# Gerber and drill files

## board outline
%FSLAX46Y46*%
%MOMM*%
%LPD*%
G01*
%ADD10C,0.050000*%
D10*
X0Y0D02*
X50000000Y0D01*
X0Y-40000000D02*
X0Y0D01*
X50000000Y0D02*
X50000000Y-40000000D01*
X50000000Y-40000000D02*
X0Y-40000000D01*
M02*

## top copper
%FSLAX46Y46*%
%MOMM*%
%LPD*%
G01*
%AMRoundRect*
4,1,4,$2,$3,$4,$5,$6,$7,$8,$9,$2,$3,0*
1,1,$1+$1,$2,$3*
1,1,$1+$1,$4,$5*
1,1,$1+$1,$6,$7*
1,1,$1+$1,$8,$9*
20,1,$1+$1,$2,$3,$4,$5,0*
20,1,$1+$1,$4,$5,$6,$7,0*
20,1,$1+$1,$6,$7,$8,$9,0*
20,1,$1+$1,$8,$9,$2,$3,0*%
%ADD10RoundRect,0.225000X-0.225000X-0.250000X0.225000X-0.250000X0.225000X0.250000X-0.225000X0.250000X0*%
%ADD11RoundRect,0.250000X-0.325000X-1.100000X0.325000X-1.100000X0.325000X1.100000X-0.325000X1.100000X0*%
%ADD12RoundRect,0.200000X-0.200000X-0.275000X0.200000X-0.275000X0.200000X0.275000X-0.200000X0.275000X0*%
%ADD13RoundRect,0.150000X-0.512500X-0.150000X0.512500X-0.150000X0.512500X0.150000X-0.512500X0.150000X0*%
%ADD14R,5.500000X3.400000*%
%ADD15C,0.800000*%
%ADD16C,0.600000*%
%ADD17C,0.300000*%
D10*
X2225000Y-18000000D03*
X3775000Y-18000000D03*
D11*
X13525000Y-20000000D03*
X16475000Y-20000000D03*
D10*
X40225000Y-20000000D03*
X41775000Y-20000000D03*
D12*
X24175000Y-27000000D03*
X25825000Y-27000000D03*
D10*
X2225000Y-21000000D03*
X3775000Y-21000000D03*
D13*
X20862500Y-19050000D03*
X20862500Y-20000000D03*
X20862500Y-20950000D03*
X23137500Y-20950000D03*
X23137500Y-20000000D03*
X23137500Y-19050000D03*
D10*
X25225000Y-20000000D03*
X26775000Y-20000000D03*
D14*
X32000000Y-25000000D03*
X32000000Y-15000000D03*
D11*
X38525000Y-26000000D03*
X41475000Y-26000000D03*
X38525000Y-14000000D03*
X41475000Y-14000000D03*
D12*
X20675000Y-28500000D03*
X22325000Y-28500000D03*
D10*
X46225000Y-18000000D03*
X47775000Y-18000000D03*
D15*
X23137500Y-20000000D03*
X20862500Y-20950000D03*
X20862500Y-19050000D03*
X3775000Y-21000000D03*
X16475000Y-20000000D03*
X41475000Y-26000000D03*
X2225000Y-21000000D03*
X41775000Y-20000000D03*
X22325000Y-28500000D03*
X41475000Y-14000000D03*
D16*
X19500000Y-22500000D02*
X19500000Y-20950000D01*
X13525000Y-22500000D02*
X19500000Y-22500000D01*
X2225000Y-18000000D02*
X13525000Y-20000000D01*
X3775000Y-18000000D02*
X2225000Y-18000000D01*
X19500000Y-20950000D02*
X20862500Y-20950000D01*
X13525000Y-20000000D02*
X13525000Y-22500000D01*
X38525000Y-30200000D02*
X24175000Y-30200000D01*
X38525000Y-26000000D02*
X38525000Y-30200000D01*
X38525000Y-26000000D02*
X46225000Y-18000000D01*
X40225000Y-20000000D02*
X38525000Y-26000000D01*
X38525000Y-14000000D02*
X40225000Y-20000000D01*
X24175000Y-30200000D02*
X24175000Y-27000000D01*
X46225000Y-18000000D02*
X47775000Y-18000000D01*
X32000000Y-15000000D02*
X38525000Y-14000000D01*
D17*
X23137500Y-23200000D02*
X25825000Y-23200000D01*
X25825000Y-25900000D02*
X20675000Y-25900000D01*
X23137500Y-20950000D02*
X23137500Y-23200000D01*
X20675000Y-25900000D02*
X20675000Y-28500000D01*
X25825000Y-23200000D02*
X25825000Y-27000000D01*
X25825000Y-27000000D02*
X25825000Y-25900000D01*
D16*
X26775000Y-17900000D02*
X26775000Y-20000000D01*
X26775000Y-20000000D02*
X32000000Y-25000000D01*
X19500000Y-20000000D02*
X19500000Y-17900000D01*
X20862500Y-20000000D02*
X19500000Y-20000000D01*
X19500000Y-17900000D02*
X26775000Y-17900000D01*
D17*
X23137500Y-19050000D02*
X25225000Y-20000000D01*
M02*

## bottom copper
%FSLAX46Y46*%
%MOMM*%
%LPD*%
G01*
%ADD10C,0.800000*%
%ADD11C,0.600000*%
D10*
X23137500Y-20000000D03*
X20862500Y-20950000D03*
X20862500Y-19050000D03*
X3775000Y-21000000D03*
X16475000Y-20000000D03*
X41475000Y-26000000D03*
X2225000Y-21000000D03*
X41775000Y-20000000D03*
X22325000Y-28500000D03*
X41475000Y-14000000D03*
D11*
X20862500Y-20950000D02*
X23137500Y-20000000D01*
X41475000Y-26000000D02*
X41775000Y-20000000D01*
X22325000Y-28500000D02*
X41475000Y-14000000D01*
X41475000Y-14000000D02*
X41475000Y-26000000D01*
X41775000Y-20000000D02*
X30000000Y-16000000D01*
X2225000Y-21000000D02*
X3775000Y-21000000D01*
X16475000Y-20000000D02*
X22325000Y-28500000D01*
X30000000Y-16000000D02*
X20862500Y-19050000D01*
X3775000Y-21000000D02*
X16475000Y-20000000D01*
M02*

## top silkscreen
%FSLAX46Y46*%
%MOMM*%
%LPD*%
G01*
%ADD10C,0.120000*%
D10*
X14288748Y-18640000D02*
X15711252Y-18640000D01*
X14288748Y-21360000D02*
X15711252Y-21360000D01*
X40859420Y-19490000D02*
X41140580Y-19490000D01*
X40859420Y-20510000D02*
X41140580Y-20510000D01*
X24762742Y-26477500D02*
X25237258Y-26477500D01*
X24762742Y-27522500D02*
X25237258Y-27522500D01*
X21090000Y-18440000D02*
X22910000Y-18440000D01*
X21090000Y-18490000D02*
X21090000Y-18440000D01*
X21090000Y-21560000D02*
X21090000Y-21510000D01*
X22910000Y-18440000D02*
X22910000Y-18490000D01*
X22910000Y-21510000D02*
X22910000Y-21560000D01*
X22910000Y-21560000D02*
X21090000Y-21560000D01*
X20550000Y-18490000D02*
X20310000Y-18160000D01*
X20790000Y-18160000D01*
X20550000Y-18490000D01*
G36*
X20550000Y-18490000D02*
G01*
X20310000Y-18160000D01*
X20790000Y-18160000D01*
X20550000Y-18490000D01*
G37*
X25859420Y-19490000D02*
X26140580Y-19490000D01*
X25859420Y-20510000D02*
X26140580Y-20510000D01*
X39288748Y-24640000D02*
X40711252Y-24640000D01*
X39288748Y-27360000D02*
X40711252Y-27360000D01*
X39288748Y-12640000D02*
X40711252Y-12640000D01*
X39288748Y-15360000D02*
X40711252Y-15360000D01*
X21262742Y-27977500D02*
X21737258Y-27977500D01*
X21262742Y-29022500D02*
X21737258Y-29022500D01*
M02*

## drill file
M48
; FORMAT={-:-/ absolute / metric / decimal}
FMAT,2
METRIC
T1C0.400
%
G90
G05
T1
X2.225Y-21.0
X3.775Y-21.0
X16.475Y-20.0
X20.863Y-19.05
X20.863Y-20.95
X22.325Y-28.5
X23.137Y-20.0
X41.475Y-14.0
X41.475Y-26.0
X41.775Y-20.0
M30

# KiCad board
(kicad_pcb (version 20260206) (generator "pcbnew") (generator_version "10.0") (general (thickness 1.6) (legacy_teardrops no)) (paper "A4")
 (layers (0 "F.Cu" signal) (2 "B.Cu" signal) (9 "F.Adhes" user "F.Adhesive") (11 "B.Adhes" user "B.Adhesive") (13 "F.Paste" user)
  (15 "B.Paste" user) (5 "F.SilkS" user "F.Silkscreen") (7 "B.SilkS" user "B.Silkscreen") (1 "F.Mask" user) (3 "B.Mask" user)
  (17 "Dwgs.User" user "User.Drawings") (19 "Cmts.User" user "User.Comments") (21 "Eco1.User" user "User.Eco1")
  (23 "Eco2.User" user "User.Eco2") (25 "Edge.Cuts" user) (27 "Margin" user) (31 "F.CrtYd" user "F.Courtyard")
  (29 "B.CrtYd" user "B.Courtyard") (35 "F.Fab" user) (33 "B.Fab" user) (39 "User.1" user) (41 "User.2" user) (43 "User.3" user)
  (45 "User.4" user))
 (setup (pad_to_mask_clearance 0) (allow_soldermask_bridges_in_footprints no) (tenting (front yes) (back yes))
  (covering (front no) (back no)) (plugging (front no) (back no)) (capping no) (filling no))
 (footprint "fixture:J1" (layer "F.Cu") (at 3 18)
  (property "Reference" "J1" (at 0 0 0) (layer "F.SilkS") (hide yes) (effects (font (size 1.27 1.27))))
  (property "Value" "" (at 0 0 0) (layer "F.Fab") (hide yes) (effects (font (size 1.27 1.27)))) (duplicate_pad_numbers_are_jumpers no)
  (pad "1" smd roundrect (at -0.775 0) (size 0.9 0.95) (layers "F.Cu" "F.Mask" "F.Paste") (roundrect_rratio 0.25) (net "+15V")
   (thermal_bridge_angle 45))
  (pad "2" smd roundrect (at 0.775 0) (size 0.9 0.95) (layers "F.Cu" "F.Mask" "F.Paste") (roundrect_rratio 0.25) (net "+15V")
   (thermal_bridge_angle 45)))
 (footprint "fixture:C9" (layer "F.Cu") (at 15 20)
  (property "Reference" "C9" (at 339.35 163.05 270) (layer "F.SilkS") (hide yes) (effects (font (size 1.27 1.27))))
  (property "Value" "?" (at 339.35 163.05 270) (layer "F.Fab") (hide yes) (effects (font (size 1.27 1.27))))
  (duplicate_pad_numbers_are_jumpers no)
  (fp_line (start -0.711252 -1.36) (end 0.711252 -1.36) (stroke (width 0.12) (type solid)) (layer "F.SilkS"))
  (fp_line (start -0.711252 1.36) (end 0.711252 1.36) (stroke (width 0.12) (type solid)) (layer "F.SilkS"))
  (pad "1" smd roundrect (at -1.475 0) (size 1.15 2.7) (layers "F.Cu" "F.Mask" "F.Paste") (roundrect_rratio 0.217391) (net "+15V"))
  (pad "2" smd roundrect (at 1.475 0) (size 1.15 2.7) (layers "F.Cu" "F.Mask" "F.Paste") (roundrect_rratio 0.217391) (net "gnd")))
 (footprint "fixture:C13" (layer "F.Cu") (at 41 20)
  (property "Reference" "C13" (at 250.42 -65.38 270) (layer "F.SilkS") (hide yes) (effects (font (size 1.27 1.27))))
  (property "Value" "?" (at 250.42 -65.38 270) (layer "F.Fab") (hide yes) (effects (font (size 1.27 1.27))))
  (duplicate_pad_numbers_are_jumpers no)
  (fp_line (start -0.14058 -0.51) (end 0.14058 -0.51) (stroke (width 0.12) (type solid)) (layer "F.SilkS"))
  (fp_line (start -0.14058 0.51) (end 0.14058 0.51) (stroke (width 0.12) (type solid)) (layer "F.SilkS"))
  (pad "1" smd roundrect (at -0.775 0) (size 0.9 0.95) (layers "F.Cu" "F.Mask" "F.Paste") (roundrect_rratio 0.25) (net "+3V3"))
  (pad "2" smd roundrect (at 0.775 0) (size 0.9 0.95) (layers "F.Cu" "F.Mask" "F.Paste") (roundrect_rratio 0.25) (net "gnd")))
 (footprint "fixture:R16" (layer "F.Cu") (at 25 27)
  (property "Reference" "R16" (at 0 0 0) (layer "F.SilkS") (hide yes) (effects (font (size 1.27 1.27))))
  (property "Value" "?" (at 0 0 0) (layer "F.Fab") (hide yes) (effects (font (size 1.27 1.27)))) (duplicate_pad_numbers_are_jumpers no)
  (fp_line (start -0.237258 -0.5225) (end 0.237258 -0.5225) (stroke (width 0.12) (type solid)) (layer "F.SilkS"))
  (fp_line (start -0.237258 0.5225) (end 0.237258 0.5225) (stroke (width 0.12) (type solid)) (layer "F.SilkS"))
  (pad "1" smd roundrect (at -0.825 0) (size 0.8 0.95) (layers "F.Cu" "F.Mask" "F.Paste") (roundrect_rratio 0.25) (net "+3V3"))
  (pad "2" smd roundrect (at 0.825 0) (size 0.8 0.95) (layers "F.Cu" "F.Mask" "F.Paste") (roundrect_rratio 0.25) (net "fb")))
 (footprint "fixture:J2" (layer "F.Cu") (at 3 21)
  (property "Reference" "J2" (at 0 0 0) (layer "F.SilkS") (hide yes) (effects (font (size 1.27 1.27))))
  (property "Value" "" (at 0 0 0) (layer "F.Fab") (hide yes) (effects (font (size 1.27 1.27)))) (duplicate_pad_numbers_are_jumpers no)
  (pad "1" smd roundrect (at -0.775 0) (size 0.9 0.95) (layers "F.Cu" "F.Mask" "F.Paste") (roundrect_rratio 0.25) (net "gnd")
   (thermal_bridge_angle 45))
  (pad "2" smd roundrect (at 0.775 0) (size 0.9 0.95) (layers "F.Cu" "F.Mask" "F.Paste") (roundrect_rratio 0.25) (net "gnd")
   (thermal_bridge_angle 45)))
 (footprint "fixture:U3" (layer "F.Cu") (at 22 20)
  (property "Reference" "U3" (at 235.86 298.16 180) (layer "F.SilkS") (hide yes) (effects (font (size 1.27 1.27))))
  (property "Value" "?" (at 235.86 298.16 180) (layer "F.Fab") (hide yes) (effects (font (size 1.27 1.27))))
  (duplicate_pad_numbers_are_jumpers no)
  (fp_line (start -0.91 -1.56) (end 0.91 -1.56) (stroke (width 0.12) (type solid)) (layer "F.SilkS"))
  (fp_line (start -0.91 -1.51) (end -0.91 -1.56) (stroke (width 0.12) (type solid)) (layer "F.SilkS"))
  (fp_line (start -0.91 1.56) (end -0.91 1.51) (stroke (width 0.12) (type solid)) (layer "F.SilkS"))
  (fp_line (start 0.91 -1.56) (end 0.91 -1.51) (stroke (width 0.12) (type solid)) (layer "F.SilkS"))
  (fp_line (start 0.91 1.51) (end 0.91 1.56) (stroke (width 0.12) (type solid)) (layer "F.SilkS"))
  (fp_line (start 0.91 1.56) (end -0.91 1.56) (stroke (width 0.12) (type solid)) (layer "F.SilkS"))
  (fp_poly (pts (xy -1.45 -1.51) (xy -1.69 -1.84) (xy -1.21 -1.84)) (stroke (width 0.12) (type solid)) (fill yes) (layer "F.SilkS"))
  (pad "1" smd roundrect (at -1.1375 -0.95) (size 1.325 0.6) (layers "F.Cu" "F.Mask" "F.Paste") (roundrect_rratio 0.25) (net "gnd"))
  (pad "2" smd roundrect (at -1.1375 0) (size 1.325 0.6) (layers "F.Cu" "F.Mask" "F.Paste") (roundrect_rratio 0.25) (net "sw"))
  (pad "3" smd roundrect (at -1.1375 0.95) (size 1.325 0.6) (layers "F.Cu" "F.Mask" "F.Paste") (roundrect_rratio 0.25) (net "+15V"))
  (pad "4" smd roundrect (at 1.1375 0.95) (size 1.325 0.6) (layers "F.Cu" "F.Mask" "F.Paste") (roundrect_rratio 0.25) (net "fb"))
  (pad "5" smd roundrect (at 1.1375 0) (size 1.325 0.6) (layers "F.Cu" "F.Mask" "F.Paste") (roundrect_rratio 0.25) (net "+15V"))
  (pad "6" smd roundrect (at 1.1375 -0.95) (size 1.325 0.6) (layers "F.Cu" "F.Mask" "F.Paste") (roundrect_rratio 0.25) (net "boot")))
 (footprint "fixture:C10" (layer "F.Cu") (at 26 20)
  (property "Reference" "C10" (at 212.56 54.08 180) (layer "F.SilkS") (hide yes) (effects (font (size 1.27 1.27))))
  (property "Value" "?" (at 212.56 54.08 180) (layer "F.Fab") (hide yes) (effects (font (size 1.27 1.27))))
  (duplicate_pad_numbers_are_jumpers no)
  (fp_line (start -0.14058 -0.51) (end 0.14058 -0.51) (stroke (width 0.12) (type solid)) (layer "F.SilkS"))
  (fp_line (start -0.14058 0.51) (end 0.14058 0.51) (stroke (width 0.12) (type solid)) (layer "F.SilkS"))
  (pad "1" smd roundrect (at -0.775 0) (size 0.9 0.95) (layers "F.Cu" "F.Mask" "F.Paste") (roundrect_rratio 0.25) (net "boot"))
  (pad "2" smd roundrect (at 0.775 0) (size 0.9 0.95) (layers "F.Cu" "F.Mask" "F.Paste") (roundrect_rratio 0.25) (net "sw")))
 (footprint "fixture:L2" (layer "F.Cu") (at 32 20 90)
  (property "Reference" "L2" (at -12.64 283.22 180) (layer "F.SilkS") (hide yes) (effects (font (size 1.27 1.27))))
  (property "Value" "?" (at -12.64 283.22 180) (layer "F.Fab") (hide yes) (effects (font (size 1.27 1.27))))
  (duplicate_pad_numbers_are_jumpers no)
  (pad "1" smd rect (at -5 0 90) (size 3.4 5.5) (layers "F.Cu" "F.Mask" "F.Paste") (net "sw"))
  (pad "2" smd rect (at 5 0 90) (size 3.4 5.5) (layers "F.Cu" "F.Mask" "F.Paste") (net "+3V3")))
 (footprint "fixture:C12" (layer "F.Cu") (at 40 26)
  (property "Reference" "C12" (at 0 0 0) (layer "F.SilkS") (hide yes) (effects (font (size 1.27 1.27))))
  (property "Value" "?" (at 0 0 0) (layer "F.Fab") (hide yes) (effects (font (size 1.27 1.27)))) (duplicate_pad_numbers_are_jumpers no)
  (fp_line (start -0.711252 -1.36) (end 0.711252 -1.36) (stroke (width 0.12) (type solid)) (layer "F.SilkS"))
  (fp_line (start -0.711252 1.36) (end 0.711252 1.36) (stroke (width 0.12) (type solid)) (layer "F.SilkS"))
  (pad "1" smd roundrect (at -1.475 0) (size 1.15 2.7) (layers "F.Cu" "F.Mask" "F.Paste") (roundrect_rratio 0.217391) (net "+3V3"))
  (pad "2" smd roundrect (at 1.475 0) (size 1.15 2.7) (layers "F.Cu" "F.Mask" "F.Paste") (roundrect_rratio 0.217391) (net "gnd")))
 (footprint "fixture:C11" (layer "F.Cu") (at 40 14)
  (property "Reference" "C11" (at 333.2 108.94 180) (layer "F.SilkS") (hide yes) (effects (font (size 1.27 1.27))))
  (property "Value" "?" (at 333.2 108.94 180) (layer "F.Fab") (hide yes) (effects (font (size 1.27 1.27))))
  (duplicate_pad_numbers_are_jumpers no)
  (fp_line (start -0.711252 -1.36) (end 0.711252 -1.36) (stroke (width 0.12) (type solid)) (layer "F.SilkS"))
  (fp_line (start -0.711252 1.36) (end 0.711252 1.36) (stroke (width 0.12) (type solid)) (layer "F.SilkS"))
  (pad "1" smd roundrect (at -1.475 0) (size 1.15 2.7) (layers "F.Cu" "F.Mask" "F.Paste") (roundrect_rratio 0.217391) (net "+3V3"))
  (pad "2" smd roundrect (at 1.475 0) (size 1.15 2.7) (layers "F.Cu" "F.Mask" "F.Paste") (roundrect_rratio 0.217391) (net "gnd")))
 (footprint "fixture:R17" (layer "F.Cu") (at 21.5 28.5)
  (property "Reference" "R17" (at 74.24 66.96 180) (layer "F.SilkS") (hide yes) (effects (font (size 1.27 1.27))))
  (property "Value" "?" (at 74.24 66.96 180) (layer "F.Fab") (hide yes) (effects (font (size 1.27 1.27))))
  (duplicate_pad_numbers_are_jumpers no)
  (fp_line (start -0.237258 -0.5225) (end 0.237258 -0.5225) (stroke (width 0.12) (type solid)) (layer "F.SilkS"))
  (fp_line (start -0.237258 0.5225) (end 0.237258 0.5225) (stroke (width 0.12) (type solid)) (layer "F.SilkS"))
  (pad "1" smd roundrect (at -0.825 0) (size 0.8 0.95) (layers "F.Cu" "F.Mask" "F.Paste") (roundrect_rratio 0.25) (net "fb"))
  (pad "2" smd roundrect (at 0.825 0) (size 0.8 0.95) (layers "F.Cu" "F.Mask" "F.Paste") (roundrect_rratio 0.25) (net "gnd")))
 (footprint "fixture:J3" (layer "F.Cu") (at 47 18)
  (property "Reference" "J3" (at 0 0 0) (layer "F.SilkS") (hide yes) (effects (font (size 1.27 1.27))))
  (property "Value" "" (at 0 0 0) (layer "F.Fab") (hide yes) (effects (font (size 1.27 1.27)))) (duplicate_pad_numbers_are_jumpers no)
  (pad "1" smd roundrect (at -0.775 0) (size 0.9 0.95) (layers "F.Cu" "F.Mask" "F.Paste") (roundrect_rratio 0.25) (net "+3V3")
   (thermal_bridge_angle 45))
  (pad "2" smd roundrect (at 0.775 0) (size 0.9 0.95) (layers "F.Cu" "F.Mask" "F.Paste") (roundrect_rratio 0.25) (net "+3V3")
   (thermal_bridge_angle 45)))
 (gr_line (start 0 0) (end 50 0) (stroke (width 0.05) (type default)) (layer "Edge.Cuts"))
 (gr_line (start 0 40) (end 0 0) (stroke (width 0.05) (type default)) (layer "Edge.Cuts"))
 (gr_line (start 50 0) (end 50 40) (stroke (width 0.05) (type default)) (layer "Edge.Cuts"))
 (gr_line (start 50 40) (end 0 40) (stroke (width 0.05) (type default)) (layer "Edge.Cuts"))
 (segment (start 19.5 22.5) (end 19.5 20.95) (width 0.6) (layer "F.Cu") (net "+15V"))
 (segment (start 13.525 22.5) (end 19.5 22.5) (width 0.6) (layer "F.Cu") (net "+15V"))
 (segment (start 2.225 18) (end 13.525 20) (width 0.6) (layer "F.Cu") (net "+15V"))
 (segment (start 3.775 18) (end 2.225 18) (width 0.6) (layer "F.Cu") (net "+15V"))
 (segment (start 19.5 20.95) (end 20.8625 20.95) (width 0.6) (layer "F.Cu") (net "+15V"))
 (segment (start 13.525 20) (end 13.525 22.5) (width 0.6) (layer "F.Cu") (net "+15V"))
 (via (at 23.1375 20) (size 0.8) (drill 0.4) (layers "F.Cu" "B.Cu") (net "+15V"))
 (via (at 20.8625 20.95) (size 0.8) (drill 0.4) (layers "F.Cu" "B.Cu") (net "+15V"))
 (segment (start 20.8625 20.95) (end 23.1375 20) (width 0.6) (layer "B.Cu") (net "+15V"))
 (via (at 20.8625 19.05) (size 0.8) (drill 0.4) (layers "F.Cu" "B.Cu") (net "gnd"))
 (via (at 3.775 21) (size 0.8) (drill 0.4) (layers "F.Cu" "B.Cu") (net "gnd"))
 (via (at 16.475 20) (size 0.8) (drill 0.4) (layers "F.Cu" "B.Cu") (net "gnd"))
 (via (at 41.475 26) (size 0.8) (drill 0.4) (layers "F.Cu" "B.Cu") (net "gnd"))
 (via (at 2.225 21) (size 0.8) (drill 0.4) (layers "F.Cu" "B.Cu") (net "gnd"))
 (via (at 41.775 20) (size 0.8) (drill 0.4) (layers "F.Cu" "B.Cu") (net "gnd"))
 (via (at 22.325 28.5) (size 0.8) (drill 0.4) (layers "F.Cu" "B.Cu") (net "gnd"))
 (segment (start 41.475 26) (end 41.775 20) (width 0.6) (layer "B.Cu") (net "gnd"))
 (segment (start 22.325 28.5) (end 41.475 14) (width 0.6) (layer "B.Cu") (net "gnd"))
 (segment (start 41.475 14) (end 41.475 26) (width 0.6) (layer "B.Cu") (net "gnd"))
 (segment (start 41.775 20) (end 30 16) (width 0.6) (layer "B.Cu") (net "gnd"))
 (segment (start 2.225 21) (end 3.775 21) (width 0.6) (layer "B.Cu") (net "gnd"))
 (segment (start 16.475 20) (end 22.325 28.5) (width 0.6) (layer "B.Cu") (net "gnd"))
 (segment (start 30 16) (end 20.8625 19.05) (width 0.6) (layer "B.Cu") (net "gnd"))
 (segment (start 3.775 21) (end 16.475 20) (width 0.6) (layer "B.Cu") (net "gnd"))
 (segment (start 38.525 30.2) (end 24.175 30.2) (width 0.6) (layer "F.Cu") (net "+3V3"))
 (segment (start 38.525 26) (end 38.525 30.2) (width 0.6) (layer "F.Cu") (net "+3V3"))
 (segment (start 38.525 26) (end 46.225 18) (width 0.6) (layer "F.Cu") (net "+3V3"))
 (segment (start 40.225 20) (end 38.525 26) (width 0.6) (layer "F.Cu") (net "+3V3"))
 (segment (start 38.525 14) (end 40.225 20) (width 0.6) (layer "F.Cu") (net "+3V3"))
 (segment (start 24.175 30.2) (end 24.175 27) (width 0.6) (layer "F.Cu") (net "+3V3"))
 (segment (start 46.225 18) (end 47.775 18) (width 0.6) (layer "F.Cu") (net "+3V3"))
 (segment (start 32 15) (end 38.525 14) (width 0.6) (layer "F.Cu") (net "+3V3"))
 (segment (start 23.1375 23.2) (end 25.825 23.2) (width 0.3) (layer "F.Cu") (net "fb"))
 (segment (start 25.825 25.9) (end 20.675 25.9) (width 0.3) (layer "F.Cu") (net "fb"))
 (segment (start 23.1375 20.95) (end 23.1375 23.2) (width 0.3) (layer "F.Cu") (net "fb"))
 (segment (start 20.675 25.9) (end 20.675 28.5) (width 0.3) (layer "F.Cu") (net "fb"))
 (segment (start 25.825 23.2) (end 25.825 27) (width 0.3) (layer "F.Cu") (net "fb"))
 (segment (start 25.825 27) (end 25.825 25.9) (width 0.3) (layer "F.Cu") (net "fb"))
 (segment (start 26.775 17.9) (end 26.775 20) (width 0.6) (layer "F.Cu") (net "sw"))
 (segment (start 26.775 20) (end 32 25) (width 0.6) (layer "F.Cu") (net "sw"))
 (segment (start 19.5 20) (end 19.5 17.9) (width 0.6) (layer "F.Cu") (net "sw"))
 (segment (start 20.8625 20) (end 19.5 20) (width 0.6) (layer "F.Cu") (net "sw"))
 (segment (start 19.5 17.9) (end 26.775 17.9) (width 0.6) (layer "F.Cu") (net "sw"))
 (via (at 41.475 14) (size 0.8) (drill 0.4) (layers "F.Cu" "B.Cu") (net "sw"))
 (segment (start 23.1375 19.05) (end 25.225 20) (width 0.3) (layer "F.Cu") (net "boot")))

